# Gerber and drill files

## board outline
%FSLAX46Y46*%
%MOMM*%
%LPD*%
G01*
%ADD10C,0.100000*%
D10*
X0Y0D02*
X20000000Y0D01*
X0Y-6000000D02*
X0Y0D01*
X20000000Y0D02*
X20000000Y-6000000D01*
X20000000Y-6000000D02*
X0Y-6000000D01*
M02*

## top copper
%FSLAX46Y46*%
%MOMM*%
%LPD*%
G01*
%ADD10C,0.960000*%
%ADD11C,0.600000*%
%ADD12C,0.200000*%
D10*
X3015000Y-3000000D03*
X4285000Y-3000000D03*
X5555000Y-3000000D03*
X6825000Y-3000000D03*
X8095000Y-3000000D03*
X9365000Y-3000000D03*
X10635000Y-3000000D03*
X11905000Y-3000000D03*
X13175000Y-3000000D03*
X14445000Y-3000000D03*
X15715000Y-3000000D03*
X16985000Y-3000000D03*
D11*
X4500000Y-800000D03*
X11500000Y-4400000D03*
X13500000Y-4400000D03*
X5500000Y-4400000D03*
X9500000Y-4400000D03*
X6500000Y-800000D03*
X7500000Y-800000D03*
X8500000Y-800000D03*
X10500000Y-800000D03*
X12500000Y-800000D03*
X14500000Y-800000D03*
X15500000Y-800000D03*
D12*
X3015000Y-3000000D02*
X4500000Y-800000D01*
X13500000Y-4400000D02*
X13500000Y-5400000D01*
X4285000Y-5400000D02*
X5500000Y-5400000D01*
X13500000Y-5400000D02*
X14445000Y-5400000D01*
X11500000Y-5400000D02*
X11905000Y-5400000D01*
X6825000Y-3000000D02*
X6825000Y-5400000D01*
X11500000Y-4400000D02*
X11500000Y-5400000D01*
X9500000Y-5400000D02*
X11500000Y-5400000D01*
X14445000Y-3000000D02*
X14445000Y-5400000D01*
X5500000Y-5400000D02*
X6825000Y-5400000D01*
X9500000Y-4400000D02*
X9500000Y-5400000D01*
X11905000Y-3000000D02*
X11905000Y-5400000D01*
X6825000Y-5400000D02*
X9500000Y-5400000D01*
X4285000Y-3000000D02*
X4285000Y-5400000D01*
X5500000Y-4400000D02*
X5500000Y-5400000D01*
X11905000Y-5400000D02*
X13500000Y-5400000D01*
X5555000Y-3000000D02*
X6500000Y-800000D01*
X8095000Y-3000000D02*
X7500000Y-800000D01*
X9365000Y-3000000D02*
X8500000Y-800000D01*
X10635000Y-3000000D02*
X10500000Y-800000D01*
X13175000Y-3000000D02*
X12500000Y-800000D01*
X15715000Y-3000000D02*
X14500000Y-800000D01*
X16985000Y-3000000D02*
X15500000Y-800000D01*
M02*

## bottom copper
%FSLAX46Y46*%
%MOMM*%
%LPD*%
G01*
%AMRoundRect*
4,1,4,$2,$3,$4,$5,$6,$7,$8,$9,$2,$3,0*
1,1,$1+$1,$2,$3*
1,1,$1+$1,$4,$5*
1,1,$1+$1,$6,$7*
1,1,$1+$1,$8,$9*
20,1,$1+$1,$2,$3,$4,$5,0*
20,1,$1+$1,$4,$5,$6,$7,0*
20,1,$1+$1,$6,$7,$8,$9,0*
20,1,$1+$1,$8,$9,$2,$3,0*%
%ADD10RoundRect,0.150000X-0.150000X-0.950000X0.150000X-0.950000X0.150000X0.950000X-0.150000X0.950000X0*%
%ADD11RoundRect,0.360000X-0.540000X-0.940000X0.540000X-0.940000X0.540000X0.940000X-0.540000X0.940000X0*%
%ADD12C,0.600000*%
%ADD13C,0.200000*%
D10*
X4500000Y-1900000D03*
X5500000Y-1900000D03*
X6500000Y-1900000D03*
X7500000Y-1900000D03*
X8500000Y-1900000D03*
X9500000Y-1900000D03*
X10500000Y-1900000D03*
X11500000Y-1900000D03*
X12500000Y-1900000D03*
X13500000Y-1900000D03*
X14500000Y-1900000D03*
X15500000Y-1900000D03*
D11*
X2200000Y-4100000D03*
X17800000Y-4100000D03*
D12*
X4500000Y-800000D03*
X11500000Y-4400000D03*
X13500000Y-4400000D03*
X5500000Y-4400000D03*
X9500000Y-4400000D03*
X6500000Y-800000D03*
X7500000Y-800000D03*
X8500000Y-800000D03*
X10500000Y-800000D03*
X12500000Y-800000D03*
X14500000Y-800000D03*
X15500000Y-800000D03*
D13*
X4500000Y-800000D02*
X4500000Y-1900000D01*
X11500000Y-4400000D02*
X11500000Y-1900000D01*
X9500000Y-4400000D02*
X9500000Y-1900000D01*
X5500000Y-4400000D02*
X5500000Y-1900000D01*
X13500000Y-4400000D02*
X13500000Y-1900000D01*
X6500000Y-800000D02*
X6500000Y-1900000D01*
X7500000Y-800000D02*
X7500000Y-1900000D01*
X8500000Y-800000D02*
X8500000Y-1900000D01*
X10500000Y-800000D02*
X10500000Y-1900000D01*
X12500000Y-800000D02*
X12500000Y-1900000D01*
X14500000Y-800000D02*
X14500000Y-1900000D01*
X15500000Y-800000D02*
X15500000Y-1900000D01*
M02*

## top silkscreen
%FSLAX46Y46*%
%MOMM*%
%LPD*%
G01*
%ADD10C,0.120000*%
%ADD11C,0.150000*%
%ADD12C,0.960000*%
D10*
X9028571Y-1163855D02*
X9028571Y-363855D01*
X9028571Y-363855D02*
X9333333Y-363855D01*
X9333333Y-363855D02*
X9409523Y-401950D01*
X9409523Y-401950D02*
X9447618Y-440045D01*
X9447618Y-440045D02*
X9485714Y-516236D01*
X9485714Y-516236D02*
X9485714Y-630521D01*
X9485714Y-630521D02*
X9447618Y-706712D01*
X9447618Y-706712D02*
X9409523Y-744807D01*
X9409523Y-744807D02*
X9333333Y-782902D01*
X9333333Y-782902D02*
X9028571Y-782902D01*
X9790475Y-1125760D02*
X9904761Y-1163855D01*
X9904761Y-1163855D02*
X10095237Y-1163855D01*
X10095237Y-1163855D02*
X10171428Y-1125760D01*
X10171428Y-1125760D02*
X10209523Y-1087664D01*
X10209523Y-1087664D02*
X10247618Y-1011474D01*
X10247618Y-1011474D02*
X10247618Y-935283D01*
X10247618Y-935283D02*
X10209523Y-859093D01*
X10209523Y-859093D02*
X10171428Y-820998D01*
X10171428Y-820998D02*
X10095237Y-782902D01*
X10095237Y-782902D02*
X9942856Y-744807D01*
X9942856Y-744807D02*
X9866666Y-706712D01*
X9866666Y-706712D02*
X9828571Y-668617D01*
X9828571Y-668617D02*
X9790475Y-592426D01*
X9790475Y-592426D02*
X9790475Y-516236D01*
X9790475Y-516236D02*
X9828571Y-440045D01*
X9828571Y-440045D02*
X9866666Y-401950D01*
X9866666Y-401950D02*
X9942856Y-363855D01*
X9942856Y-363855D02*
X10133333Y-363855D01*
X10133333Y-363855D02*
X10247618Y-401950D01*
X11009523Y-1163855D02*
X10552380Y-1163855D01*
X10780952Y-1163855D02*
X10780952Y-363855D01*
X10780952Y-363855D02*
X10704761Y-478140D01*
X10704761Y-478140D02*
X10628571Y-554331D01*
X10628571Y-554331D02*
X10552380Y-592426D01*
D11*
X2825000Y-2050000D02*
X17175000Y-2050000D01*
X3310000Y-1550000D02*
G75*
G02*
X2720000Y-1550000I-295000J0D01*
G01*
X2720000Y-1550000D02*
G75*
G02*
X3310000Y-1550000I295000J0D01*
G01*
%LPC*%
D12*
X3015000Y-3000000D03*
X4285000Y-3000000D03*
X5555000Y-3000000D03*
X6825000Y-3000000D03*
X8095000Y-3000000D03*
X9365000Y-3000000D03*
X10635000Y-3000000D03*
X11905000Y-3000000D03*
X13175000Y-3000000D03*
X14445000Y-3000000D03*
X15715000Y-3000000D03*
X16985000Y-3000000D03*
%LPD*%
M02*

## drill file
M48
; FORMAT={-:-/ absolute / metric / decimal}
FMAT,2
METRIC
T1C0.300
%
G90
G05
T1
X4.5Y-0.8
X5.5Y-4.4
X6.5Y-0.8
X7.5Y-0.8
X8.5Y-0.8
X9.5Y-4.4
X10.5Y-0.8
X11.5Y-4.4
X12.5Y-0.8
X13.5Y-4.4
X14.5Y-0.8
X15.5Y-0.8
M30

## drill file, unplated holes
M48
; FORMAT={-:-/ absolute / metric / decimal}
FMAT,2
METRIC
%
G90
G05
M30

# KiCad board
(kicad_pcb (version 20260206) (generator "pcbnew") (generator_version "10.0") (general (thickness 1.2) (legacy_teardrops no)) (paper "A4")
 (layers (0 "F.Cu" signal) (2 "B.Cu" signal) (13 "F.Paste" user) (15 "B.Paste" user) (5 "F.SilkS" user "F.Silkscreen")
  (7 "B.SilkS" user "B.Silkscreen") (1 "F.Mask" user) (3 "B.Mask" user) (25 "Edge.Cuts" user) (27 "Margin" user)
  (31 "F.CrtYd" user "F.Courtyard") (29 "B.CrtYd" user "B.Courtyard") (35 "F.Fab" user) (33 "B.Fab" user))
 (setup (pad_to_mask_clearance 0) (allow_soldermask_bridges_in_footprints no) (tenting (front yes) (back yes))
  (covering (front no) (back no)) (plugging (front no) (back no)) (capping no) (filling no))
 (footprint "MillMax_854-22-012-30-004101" (layer "F.Cu") (at 10 3)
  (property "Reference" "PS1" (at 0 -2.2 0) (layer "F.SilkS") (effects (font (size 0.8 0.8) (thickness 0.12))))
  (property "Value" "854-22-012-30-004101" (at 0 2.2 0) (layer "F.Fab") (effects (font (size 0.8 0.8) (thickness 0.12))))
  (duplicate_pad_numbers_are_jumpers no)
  (fp_line (start -7.175 -0.95) (end 7.175 -0.95) (stroke (width 0.15) (type solid)) (layer "F.SilkS"))
  (fp_circle (center -6.985 -1.45) (end -6.69 -1.45) (stroke (width 0.15) (type solid)) (fill no) (layer "F.SilkS"))
  (pad "1" smd circle (at -6.985 0) (size 0.96 0.96) (layers "F.Cu" "F.Mask" "F.Paste") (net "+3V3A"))
  (pad "2" smd circle (at -5.715 0) (size 0.96 0.96) (layers "F.Cu" "F.Mask" "F.Paste") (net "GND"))
  (pad "3" smd circle (at -4.445 0) (size 0.96 0.96) (layers "F.Cu" "F.Mask" "F.Paste") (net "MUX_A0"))
  (pad "4" smd circle (at -3.175 0) (size 0.96 0.96) (layers "F.Cu" "F.Mask" "F.Paste") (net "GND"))
  (pad "5" smd circle (at -1.905 0) (size 0.96 0.96) (layers "F.Cu" "F.Mask" "F.Paste") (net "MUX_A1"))
  (pad "6" smd circle (at -0.635 0) (size 0.96 0.96) (layers "F.Cu" "F.Mask" "F.Paste") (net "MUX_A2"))
  (pad "7" smd circle (at 0.635 0) (size 0.96 0.96) (layers "F.Cu" "F.Mask" "F.Paste") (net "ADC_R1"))
  (pad "8" smd circle (at 1.905 0) (size 0.96 0.96) (layers "F.Cu" "F.Mask" "F.Paste") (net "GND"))
  (pad "9" smd circle (at 3.175 0) (size 0.96 0.96) (layers "F.Cu" "F.Mask" "F.Paste") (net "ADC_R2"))
  (pad "10" smd circle (at 4.445 0) (size 0.96 0.96) (layers "F.Cu" "F.Mask" "F.Paste") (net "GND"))
  (pad "11" smd circle (at 5.715 0) (size 0.96 0.96) (layers "F.Cu" "F.Mask" "F.Paste") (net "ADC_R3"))
  (pad "12" smd circle (at 6.985 0) (size 0.96 0.96) (layers "F.Cu" "F.Mask" "F.Paste") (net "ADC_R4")))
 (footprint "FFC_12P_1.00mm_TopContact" (layer "B.Cu") (at 10 3)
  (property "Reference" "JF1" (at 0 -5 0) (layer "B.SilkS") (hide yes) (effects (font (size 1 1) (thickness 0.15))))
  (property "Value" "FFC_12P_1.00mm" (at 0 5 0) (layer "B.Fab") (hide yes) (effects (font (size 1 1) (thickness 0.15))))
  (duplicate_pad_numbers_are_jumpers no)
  (pad "1" smd roundrect (at -5.5 -1.1) (size 0.6 2.2) (layers "B.Cu" "B.Mask" "B.Paste") (roundrect_rratio 0.25) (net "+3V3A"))
  (pad "2" smd roundrect (at -4.5 -1.1) (size 0.6 2.2) (layers "B.Cu" "B.Mask" "B.Paste") (roundrect_rratio 0.25) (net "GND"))
  (pad "3" smd roundrect (at -3.5 -1.1) (size 0.6 2.2) (layers "B.Cu" "B.Mask" "B.Paste") (roundrect_rratio 0.25) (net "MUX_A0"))
  (pad "4" smd roundrect (at -2.5 -1.1) (size 0.6 2.2) (layers "B.Cu" "B.Mask" "B.Paste") (roundrect_rratio 0.25) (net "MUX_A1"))
  (pad "5" smd roundrect (at -1.5 -1.1) (size 0.6 2.2) (layers "B.Cu" "B.Mask" "B.Paste") (roundrect_rratio 0.25) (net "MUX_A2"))
  (pad "6" smd roundrect (at -0.5 -1.1) (size 0.6 2.2) (layers "B.Cu" "B.Mask" "B.Paste") (roundrect_rratio 0.25) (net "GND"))
  (pad "7" smd roundrect (at 0.5 -1.1) (size 0.6 2.2) (layers "B.Cu" "B.Mask" "B.Paste") (roundrect_rratio 0.25) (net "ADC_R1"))
  (pad "8" smd roundrect (at 1.5 -1.1) (size 0.6 2.2) (layers "B.Cu" "B.Mask" "B.Paste") (roundrect_rratio 0.25) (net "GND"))
  (pad "9" smd roundrect (at 2.5 -1.1) (size 0.6 2.2) (layers "B.Cu" "B.Mask" "B.Paste") (roundrect_rratio 0.25) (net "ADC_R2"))
  (pad "10" smd roundrect (at 3.5 -1.1) (size 0.6 2.2) (layers "B.Cu" "B.Mask" "B.Paste") (roundrect_rratio 0.25) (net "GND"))
  (pad "11" smd roundrect (at 4.5 -1.1) (size 0.6 2.2) (layers "B.Cu" "B.Mask" "B.Paste") (roundrect_rratio 0.25) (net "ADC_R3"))
  (pad "12" smd roundrect (at 5.5 -1.1) (size 0.6 2.2) (layers "B.Cu" "B.Mask" "B.Paste") (roundrect_rratio 0.25) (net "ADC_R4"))
  (pad "MP" smd roundrect (at -7.8 1.1) (size 1.8 2.6) (layers "B.Cu" "B.Mask" "B.Paste") (roundrect_rratio 0.2))
  (pad "MP" smd roundrect (at 7.8 1.1) (size 1.8 2.6) (layers "B.Cu" "B.Mask" "B.Paste") (roundrect_rratio 0.2)))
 (gr_line (start 0 0) (end 20 0) (stroke (width 0.1) (type solid)) (layer "Edge.Cuts"))
 (gr_line (start 0 6) (end 0 0) (stroke (width 0.1) (type solid)) (layer "Edge.Cuts"))
 (gr_line (start 20 0) (end 20 6) (stroke (width 0.1) (type solid)) (layer "Edge.Cuts"))
 (gr_line (start 20 6) (end 0 6) (stroke (width 0.1) (type solid)) (layer "Edge.Cuts"))
 (segment (start 3.015 3) (end 4.5 0.8) (width 0.2) (layer "F.Cu") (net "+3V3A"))
 (via (at 4.5 0.8) (size 0.6) (drill 0.3) (layers "F.Cu" "B.Cu") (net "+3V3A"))
 (segment (start 4.5 0.8) (end 4.5 1.9) (width 0.2) (layer "B.Cu") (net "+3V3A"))
 (segment (start 13.5 4.4) (end 13.5 5.4) (width 0.2) (layer "F.Cu") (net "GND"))
 (segment (start 4.285 5.4) (end 5.5 5.4) (width 0.2) (layer "F.Cu") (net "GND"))
 (segment (start 13.5 5.4) (end 14.445 5.4) (width 0.2) (layer "F.Cu") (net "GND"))
 (segment (start 11.5 5.4) (end 11.905 5.4) (width 0.2) (layer "F.Cu") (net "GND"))
 (segment (start 6.825 3) (end 6.825 5.4) (width 0.2) (layer "F.Cu") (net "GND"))
 (segment (start 11.5 4.4) (end 11.5 5.4) (width 0.2) (layer "F.Cu") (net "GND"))
 (segment (start 9.5 5.4) (end 11.5 5.4) (width 0.2) (layer "F.Cu") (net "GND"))
 (segment (start 14.445 3) (end 14.445 5.4) (width 0.2) (layer "F.Cu") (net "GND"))
 (segment (start 5.5 5.4) (end 6.825 5.4) (width 0.2) (layer "F.Cu") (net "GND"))
 (segment (start 9.5 4.4) (end 9.5 5.4) (width 0.2) (layer "F.Cu") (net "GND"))
 (segment (start 11.905 3) (end 11.905 5.4) (width 0.2) (layer "F.Cu") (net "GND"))
 (segment (start 6.825 5.4) (end 9.5 5.4) (width 0.2) (layer "F.Cu") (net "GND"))
 (segment (start 4.285 3) (end 4.285 5.4) (width 0.2) (layer "F.Cu") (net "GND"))
 (segment (start 5.5 4.4) (end 5.5 5.4) (width 0.2) (layer "F.Cu") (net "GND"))
 (segment (start 11.905 5.4) (end 13.5 5.4) (width 0.2) (layer "F.Cu") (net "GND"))
 (via (at 11.5 4.4) (size 0.6) (drill 0.3) (layers "F.Cu" "B.Cu") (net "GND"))
 (via (at 13.5 4.4) (size 0.6) (drill 0.3) (layers "F.Cu" "B.Cu") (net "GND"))
 (via (at 5.5 4.4) (size 0.6) (drill 0.3) (layers "F.Cu" "B.Cu") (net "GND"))
 (via (at 9.5 4.4) (size 0.6) (drill 0.3) (layers "F.Cu" "B.Cu") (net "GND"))
 (segment (start 11.5 4.4) (end 11.5 1.9) (width 0.2) (layer "B.Cu") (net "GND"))
 (segment (start 9.5 4.4) (end 9.5 1.9) (width 0.2) (layer "B.Cu") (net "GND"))
 (segment (start 5.5 4.4) (end 5.5 1.9) (width 0.2) (layer "B.Cu") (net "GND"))
 (segment (start 13.5 4.4) (end 13.5 1.9) (width 0.2) (layer "B.Cu") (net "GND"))
 (segment (start 5.555 3) (end 6.5 0.8) (width 0.2) (layer "F.Cu") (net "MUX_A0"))
 (via (at 6.5 0.8) (size 0.6) (drill 0.3) (layers "F.Cu" "B.Cu") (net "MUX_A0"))
 (segment (start 6.5 0.8) (end 6.5 1.9) (width 0.2) (layer "B.Cu") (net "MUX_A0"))
 (segment (start 8.095 3) (end 7.5 0.8) (width 0.2) (layer "F.Cu") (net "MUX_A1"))
 (via (at 7.5 0.8) (size 0.6) (drill 0.3) (layers "F.Cu" "B.Cu") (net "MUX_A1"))
 (segment (start 7.5 0.8) (end 7.5 1.9) (width 0.2) (layer "B.Cu") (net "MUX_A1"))
 (segment (start 9.365 3) (end 8.5 0.8) (width 0.2) (layer "F.Cu") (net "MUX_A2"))
 (via (at 8.5 0.8) (size 0.6) (drill 0.3) (layers "F.Cu" "B.Cu") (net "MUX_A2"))
 (segment (start 8.5 0.8) (end 8.5 1.9) (width 0.2) (layer "B.Cu") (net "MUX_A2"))
 (segment (start 10.635 3) (end 10.5 0.8) (width 0.2) (layer "F.Cu") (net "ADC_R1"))
 (via (at 10.5 0.8) (size 0.6) (drill 0.3) (layers "F.Cu" "B.Cu") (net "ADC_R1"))
 (segment (start 10.5 0.8) (end 10.5 1.9) (width 0.2) (layer "B.Cu") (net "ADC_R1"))
 (segment (start 13.175 3) (end 12.5 0.8) (width 0.2) (layer "F.Cu") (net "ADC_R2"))
 (via (at 12.5 0.8) (size 0.6) (drill 0.3) (layers "F.Cu" "B.Cu") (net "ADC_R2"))
 (segment (start 12.5 0.8) (end 12.5 1.9) (width 0.2) (layer "B.Cu") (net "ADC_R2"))
 (segment (start 15.715 3) (end 14.5 0.8) (width 0.2) (layer "F.Cu") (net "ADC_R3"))
 (via (at 14.5 0.8) (size 0.6) (drill 0.3) (layers "F.Cu" "B.Cu") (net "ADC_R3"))
 (segment (start 14.5 0.8) (end 14.5 1.9) (width 0.2) (layer "B.Cu") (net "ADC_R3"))
 (segment (start 16.985 3) (end 15.5 0.8) (width 0.2) (layer "F.Cu") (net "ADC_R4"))
 (via (at 15.5 0.8) (size 0.6) (drill 0.3) (layers "F.Cu" "B.Cu") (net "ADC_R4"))
 (segment (start 15.5 0.8) (end 15.5 1.9) (width 0.2) (layer "B.Cu") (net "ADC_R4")))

